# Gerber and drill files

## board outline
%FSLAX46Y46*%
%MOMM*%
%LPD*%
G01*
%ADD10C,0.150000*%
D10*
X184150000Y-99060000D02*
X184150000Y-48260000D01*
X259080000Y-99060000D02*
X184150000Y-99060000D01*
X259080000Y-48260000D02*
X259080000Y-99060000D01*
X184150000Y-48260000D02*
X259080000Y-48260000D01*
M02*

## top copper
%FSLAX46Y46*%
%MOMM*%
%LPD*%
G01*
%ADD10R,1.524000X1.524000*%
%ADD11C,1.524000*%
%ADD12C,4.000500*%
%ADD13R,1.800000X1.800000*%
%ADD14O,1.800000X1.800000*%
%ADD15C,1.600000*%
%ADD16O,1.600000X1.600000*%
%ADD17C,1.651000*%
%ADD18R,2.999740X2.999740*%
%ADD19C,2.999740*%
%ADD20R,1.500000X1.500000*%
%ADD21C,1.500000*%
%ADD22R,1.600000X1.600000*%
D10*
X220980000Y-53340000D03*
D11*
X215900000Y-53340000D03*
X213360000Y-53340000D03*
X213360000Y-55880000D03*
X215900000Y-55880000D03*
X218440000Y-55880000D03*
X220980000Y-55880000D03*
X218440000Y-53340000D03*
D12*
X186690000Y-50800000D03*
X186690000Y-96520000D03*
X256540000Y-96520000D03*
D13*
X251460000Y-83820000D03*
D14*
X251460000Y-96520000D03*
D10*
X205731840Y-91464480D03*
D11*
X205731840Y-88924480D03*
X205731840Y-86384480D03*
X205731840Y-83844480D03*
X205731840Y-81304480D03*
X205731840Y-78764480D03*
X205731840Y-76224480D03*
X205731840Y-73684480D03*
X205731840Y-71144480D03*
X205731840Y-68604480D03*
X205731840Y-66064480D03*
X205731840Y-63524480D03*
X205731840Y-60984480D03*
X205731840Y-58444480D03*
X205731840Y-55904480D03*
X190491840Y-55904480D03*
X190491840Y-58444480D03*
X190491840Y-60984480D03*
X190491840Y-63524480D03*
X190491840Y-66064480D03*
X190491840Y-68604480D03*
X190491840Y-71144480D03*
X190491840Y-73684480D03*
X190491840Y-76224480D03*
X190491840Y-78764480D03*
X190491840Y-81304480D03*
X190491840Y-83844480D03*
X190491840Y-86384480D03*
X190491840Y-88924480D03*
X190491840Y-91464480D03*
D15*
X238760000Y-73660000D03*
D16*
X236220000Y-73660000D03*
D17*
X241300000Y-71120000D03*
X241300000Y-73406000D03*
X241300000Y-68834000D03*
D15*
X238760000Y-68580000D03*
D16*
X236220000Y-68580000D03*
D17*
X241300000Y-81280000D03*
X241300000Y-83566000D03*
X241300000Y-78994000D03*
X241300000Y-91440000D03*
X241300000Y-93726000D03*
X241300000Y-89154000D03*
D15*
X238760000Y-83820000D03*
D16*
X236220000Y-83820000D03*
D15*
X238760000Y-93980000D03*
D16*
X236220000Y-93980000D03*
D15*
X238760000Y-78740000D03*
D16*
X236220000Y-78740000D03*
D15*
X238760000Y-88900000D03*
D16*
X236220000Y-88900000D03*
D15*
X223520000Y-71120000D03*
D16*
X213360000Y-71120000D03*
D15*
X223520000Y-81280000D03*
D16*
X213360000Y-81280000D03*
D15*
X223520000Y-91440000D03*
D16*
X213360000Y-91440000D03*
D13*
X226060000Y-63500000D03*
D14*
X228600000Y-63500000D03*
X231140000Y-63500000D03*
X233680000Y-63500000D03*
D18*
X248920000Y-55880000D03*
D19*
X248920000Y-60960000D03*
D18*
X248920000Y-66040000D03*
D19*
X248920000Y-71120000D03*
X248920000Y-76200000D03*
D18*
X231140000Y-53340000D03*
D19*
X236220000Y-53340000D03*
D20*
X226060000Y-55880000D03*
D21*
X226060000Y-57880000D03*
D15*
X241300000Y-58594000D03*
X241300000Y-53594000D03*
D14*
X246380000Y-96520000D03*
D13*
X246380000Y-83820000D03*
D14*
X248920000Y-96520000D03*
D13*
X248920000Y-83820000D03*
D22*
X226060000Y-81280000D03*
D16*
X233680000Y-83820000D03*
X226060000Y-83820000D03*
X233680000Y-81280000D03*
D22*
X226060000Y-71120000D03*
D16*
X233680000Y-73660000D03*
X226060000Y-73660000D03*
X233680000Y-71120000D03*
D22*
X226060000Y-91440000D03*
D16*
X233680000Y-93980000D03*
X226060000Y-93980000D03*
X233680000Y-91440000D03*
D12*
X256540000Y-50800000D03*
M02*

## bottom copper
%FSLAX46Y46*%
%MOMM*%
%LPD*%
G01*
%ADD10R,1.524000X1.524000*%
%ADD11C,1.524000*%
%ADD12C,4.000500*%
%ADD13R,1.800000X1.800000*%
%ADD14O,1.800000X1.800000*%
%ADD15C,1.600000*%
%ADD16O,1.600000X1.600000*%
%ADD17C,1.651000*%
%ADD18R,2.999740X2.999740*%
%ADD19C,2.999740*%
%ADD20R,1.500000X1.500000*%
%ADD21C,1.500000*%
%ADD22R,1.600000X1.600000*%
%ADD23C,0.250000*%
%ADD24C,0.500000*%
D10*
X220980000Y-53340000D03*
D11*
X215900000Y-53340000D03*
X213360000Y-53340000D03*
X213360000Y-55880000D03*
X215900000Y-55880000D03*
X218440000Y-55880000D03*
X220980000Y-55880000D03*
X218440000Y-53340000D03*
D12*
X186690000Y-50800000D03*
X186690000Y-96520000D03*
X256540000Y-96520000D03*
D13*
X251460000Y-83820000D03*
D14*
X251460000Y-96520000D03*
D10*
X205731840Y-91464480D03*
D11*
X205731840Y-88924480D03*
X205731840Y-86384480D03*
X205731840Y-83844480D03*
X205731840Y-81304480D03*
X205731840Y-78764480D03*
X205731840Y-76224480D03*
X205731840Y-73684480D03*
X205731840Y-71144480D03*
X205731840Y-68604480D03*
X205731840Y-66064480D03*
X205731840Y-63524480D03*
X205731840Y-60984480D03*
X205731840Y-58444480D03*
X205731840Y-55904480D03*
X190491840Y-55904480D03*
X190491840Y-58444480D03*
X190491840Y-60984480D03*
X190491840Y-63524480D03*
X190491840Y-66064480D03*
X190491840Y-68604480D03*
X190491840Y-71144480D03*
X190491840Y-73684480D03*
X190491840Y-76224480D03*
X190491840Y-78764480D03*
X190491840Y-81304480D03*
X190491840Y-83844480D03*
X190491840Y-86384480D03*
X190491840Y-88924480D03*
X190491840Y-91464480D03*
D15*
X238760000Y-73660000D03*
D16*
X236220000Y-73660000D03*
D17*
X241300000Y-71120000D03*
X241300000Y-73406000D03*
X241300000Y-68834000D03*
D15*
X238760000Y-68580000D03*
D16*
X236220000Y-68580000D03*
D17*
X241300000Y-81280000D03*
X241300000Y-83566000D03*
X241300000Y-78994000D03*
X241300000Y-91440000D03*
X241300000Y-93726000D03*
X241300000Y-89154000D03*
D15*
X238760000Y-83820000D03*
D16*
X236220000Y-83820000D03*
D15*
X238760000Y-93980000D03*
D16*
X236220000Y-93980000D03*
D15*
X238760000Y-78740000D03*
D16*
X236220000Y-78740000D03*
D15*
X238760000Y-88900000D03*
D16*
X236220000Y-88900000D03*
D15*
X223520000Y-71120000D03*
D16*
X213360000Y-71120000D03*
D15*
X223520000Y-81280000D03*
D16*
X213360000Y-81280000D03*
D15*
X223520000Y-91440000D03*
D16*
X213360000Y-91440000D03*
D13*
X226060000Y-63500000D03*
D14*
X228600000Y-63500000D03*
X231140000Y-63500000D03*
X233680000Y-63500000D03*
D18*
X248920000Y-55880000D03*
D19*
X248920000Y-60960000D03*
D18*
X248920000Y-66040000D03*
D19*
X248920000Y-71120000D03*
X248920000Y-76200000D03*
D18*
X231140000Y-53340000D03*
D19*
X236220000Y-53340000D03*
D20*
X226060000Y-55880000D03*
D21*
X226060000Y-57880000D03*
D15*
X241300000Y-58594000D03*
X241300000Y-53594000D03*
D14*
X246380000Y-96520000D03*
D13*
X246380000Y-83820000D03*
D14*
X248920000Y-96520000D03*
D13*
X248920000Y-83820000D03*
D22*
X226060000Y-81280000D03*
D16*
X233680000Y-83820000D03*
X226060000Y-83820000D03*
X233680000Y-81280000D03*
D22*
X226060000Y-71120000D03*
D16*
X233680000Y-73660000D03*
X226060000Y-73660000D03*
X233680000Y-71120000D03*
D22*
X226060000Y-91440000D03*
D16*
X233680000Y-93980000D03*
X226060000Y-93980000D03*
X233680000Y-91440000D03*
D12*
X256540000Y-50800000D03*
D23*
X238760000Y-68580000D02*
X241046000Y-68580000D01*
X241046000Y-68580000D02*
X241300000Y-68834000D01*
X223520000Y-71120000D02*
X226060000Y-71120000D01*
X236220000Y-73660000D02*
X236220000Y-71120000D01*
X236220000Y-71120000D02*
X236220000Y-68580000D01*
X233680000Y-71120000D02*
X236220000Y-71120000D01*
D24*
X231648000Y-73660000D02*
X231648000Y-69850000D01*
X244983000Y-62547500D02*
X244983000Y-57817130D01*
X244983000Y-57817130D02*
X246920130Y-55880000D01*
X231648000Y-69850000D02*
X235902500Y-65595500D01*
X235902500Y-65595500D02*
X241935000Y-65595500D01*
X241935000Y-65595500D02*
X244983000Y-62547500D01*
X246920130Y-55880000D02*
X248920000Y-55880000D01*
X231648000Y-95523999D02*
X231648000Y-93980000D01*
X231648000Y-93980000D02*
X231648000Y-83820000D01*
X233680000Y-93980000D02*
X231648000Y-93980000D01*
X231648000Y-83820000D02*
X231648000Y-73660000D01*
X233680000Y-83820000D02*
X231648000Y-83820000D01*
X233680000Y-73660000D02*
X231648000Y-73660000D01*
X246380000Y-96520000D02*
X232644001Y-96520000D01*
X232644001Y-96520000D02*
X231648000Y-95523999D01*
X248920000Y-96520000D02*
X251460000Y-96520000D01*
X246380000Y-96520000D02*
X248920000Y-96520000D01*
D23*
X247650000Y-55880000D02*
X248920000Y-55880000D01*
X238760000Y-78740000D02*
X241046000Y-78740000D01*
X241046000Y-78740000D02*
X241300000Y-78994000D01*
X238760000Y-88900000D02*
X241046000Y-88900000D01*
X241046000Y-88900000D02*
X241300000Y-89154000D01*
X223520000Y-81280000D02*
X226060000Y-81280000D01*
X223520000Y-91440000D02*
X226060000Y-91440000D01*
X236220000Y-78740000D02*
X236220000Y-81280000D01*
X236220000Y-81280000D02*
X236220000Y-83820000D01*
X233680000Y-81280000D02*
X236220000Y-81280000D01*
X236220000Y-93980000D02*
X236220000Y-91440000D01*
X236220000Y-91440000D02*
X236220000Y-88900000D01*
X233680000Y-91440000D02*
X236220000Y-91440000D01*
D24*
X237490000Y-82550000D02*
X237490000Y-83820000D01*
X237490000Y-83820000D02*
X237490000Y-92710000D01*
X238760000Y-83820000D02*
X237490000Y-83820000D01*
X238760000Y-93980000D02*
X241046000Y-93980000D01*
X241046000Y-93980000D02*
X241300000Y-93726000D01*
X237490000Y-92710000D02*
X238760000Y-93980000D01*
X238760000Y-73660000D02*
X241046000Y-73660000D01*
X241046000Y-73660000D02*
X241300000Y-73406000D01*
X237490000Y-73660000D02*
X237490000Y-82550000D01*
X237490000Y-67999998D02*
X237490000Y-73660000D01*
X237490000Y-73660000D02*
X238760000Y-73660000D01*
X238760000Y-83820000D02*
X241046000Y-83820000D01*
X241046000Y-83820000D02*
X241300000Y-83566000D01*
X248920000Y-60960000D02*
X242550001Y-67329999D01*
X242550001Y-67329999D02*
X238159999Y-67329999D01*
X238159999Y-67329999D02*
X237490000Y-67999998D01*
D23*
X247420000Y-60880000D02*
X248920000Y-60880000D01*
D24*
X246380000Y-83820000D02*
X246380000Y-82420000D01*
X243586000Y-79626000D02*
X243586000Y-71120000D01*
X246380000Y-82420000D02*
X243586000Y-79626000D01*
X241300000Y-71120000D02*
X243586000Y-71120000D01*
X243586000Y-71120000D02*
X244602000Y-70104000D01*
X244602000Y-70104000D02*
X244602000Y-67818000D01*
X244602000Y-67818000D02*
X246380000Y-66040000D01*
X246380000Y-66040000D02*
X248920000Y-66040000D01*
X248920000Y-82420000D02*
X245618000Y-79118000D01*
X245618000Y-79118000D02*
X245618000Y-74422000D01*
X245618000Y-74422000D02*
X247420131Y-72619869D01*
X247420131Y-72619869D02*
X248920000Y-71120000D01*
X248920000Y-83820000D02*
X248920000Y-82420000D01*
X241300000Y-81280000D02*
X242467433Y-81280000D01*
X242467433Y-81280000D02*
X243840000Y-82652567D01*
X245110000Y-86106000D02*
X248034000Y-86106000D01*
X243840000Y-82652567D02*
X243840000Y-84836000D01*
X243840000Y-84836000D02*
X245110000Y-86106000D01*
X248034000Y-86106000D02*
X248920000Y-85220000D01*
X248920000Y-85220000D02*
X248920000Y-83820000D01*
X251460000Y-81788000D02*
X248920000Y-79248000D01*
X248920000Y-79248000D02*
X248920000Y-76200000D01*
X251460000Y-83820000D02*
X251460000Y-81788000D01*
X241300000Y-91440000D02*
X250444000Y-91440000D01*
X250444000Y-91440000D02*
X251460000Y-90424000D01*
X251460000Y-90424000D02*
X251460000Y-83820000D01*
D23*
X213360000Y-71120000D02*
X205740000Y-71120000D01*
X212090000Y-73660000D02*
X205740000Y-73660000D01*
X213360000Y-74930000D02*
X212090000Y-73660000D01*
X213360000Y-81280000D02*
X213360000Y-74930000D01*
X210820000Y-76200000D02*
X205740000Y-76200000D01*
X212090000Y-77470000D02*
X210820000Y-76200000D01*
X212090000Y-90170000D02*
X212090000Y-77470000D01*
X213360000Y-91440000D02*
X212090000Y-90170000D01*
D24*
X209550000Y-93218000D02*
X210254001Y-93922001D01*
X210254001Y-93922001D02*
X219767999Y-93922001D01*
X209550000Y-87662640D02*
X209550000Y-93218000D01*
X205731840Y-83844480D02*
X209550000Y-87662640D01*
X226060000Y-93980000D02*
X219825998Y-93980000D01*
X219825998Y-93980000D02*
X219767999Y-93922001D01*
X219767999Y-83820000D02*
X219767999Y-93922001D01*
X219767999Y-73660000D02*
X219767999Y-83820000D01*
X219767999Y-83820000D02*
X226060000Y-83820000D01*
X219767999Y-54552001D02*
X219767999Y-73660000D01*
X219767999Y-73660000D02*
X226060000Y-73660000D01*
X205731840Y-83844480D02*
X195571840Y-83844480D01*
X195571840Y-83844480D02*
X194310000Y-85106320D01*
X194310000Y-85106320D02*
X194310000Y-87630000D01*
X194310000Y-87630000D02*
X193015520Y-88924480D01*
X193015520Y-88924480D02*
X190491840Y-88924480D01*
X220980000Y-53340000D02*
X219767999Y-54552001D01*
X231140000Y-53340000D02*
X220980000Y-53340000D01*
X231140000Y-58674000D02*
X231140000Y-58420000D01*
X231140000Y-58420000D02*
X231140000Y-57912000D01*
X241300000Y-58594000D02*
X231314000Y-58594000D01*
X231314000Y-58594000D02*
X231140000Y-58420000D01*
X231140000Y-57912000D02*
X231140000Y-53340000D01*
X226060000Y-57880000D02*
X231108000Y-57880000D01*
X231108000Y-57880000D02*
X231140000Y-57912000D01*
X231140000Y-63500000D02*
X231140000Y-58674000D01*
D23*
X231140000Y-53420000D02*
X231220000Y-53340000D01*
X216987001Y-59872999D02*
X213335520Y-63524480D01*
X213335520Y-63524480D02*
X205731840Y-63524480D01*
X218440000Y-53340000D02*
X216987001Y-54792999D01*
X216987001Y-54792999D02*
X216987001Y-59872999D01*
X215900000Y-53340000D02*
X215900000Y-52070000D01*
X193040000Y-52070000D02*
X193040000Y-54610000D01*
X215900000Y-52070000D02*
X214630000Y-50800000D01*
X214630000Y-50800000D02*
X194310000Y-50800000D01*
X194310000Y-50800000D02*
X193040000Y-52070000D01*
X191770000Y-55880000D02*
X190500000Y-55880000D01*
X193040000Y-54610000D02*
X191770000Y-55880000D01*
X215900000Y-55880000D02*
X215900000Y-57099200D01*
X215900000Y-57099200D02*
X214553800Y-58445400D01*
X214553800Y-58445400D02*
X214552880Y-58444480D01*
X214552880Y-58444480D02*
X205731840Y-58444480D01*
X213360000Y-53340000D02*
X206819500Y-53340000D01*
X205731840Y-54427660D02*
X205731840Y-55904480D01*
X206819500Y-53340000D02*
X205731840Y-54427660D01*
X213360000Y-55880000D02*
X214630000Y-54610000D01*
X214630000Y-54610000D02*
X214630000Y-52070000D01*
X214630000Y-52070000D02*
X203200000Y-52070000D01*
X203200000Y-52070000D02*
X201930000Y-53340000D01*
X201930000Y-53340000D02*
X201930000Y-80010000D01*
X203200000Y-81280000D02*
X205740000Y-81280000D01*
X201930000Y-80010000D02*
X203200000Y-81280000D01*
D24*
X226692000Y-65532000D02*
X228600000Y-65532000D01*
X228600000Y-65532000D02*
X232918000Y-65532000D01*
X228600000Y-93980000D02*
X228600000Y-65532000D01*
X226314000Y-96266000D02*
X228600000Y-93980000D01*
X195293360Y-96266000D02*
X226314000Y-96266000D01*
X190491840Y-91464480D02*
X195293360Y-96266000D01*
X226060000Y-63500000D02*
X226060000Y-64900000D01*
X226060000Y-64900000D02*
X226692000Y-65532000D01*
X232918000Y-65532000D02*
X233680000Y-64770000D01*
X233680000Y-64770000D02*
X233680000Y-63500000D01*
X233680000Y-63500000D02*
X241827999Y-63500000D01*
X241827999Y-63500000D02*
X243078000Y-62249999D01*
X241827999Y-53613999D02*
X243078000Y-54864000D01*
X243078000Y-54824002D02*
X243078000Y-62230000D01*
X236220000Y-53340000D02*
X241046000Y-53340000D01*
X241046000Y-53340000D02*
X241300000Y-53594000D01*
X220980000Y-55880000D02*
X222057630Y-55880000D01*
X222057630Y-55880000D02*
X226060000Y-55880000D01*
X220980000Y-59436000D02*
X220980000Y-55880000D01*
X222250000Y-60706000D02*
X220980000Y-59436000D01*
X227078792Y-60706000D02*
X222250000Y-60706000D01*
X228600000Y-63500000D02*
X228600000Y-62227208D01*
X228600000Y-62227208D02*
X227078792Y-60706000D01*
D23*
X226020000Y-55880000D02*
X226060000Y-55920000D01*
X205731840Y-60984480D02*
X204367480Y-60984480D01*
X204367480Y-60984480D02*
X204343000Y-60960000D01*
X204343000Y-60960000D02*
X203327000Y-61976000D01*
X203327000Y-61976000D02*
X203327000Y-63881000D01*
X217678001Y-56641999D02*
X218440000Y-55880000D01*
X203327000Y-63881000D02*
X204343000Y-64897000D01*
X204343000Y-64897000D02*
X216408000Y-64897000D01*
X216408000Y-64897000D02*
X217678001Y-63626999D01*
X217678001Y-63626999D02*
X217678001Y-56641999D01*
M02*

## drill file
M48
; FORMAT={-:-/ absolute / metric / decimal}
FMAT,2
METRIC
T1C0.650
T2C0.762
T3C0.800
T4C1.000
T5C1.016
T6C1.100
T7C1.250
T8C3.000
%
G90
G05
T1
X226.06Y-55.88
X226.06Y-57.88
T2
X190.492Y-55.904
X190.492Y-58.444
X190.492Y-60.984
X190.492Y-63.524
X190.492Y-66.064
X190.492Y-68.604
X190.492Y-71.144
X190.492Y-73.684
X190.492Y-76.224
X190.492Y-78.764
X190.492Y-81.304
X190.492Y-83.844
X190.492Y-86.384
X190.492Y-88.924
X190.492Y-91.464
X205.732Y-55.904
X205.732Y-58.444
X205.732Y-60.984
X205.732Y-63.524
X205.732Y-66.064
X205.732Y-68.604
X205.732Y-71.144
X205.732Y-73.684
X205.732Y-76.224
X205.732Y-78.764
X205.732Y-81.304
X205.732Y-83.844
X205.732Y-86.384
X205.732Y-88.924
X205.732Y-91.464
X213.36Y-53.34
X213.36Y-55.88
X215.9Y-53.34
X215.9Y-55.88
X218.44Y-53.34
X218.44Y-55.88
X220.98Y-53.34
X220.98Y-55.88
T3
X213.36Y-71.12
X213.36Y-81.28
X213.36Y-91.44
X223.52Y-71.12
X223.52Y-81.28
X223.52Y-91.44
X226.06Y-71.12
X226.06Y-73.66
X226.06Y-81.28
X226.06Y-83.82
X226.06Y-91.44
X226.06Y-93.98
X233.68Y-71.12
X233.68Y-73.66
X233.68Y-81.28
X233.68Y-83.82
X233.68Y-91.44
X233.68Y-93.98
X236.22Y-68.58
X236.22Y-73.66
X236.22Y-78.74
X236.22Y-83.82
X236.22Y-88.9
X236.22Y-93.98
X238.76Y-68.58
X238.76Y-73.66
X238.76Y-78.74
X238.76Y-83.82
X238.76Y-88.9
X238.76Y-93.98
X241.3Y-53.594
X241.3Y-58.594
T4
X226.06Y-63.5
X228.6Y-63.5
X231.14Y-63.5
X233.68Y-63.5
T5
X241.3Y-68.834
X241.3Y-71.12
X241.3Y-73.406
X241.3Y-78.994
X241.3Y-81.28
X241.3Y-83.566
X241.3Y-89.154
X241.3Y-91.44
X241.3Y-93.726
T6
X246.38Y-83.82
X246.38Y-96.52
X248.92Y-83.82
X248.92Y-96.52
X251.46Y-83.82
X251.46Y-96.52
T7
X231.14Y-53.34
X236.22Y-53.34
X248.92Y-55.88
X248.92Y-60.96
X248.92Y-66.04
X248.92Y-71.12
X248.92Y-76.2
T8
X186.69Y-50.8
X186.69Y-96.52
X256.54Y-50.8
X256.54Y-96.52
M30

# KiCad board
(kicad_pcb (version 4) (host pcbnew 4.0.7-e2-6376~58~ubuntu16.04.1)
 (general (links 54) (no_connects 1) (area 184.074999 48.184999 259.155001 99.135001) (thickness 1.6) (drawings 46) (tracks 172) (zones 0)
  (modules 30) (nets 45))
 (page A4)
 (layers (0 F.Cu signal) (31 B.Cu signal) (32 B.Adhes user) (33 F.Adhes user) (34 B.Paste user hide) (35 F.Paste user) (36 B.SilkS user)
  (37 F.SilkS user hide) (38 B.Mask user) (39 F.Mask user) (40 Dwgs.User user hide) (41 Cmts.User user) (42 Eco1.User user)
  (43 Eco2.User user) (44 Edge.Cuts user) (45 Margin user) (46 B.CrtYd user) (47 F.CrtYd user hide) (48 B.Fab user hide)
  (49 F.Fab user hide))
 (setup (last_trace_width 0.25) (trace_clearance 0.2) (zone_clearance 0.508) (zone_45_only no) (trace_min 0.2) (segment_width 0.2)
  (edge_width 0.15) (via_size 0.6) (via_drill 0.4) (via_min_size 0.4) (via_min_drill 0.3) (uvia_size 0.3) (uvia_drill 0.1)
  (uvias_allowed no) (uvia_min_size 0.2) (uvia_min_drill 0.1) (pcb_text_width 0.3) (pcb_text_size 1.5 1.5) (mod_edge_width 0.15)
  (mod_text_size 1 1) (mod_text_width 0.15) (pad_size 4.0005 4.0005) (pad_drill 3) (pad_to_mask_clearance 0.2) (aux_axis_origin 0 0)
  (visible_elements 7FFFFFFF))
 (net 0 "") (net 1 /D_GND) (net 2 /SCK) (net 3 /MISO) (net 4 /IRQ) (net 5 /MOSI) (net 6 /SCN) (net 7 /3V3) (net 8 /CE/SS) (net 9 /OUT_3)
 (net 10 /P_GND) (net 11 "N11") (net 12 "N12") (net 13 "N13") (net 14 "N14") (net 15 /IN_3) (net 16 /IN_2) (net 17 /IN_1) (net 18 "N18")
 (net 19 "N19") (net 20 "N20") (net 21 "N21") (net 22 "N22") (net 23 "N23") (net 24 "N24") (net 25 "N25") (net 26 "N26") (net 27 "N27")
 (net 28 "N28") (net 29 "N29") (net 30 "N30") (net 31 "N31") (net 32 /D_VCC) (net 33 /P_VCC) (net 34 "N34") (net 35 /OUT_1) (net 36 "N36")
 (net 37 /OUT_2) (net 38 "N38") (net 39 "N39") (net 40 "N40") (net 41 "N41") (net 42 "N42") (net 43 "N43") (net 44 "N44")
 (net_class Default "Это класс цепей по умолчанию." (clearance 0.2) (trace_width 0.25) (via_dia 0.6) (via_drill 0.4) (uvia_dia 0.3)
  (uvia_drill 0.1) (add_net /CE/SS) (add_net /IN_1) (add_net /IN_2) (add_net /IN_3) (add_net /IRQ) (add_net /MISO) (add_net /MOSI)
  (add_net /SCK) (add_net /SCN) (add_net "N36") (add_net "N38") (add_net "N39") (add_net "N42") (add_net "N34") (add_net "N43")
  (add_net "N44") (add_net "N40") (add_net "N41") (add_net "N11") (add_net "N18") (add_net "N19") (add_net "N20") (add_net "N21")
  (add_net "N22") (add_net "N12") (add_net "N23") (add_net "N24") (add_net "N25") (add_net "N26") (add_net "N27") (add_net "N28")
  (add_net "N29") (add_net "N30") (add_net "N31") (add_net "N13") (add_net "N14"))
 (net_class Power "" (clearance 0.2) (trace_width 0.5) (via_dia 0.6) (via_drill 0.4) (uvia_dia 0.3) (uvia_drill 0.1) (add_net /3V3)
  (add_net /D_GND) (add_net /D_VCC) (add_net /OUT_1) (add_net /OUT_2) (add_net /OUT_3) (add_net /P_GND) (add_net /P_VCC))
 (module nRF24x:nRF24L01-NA (layer F.Cu) (at 215.265 67.31)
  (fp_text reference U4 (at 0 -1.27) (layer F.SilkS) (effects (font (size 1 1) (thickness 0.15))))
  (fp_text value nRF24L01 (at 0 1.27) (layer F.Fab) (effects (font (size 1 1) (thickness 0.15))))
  (pad 1 thru_hole rect (at 5.715 -13.97) (size 1.524 1.524) (drill 0.762) (layers *.Cu *.Mask) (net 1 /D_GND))
  (pad 5 thru_hole circle (at 0.635 -13.97) (size 1.524 1.524) (drill 0.762) (layers *.Cu *.Mask) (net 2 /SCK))
  (pad 7 thru_hole circle (at -1.905 -13.97) (size 1.524 1.524) (drill 0.762) (layers *.Cu *.Mask) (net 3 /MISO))
  (pad 8 thru_hole circle (at -1.905 -11.43) (size 1.524 1.524) (drill 0.762) (layers *.Cu *.Mask) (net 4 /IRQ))
  (pad 6 thru_hole circle (at 0.635 -11.43) (size 1.524 1.524) (drill 0.762) (layers *.Cu *.Mask) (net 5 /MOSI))
  (pad 4 thru_hole circle (at 3.175 -11.43) (size 1.524 1.524) (drill 0.762) (layers *.Cu *.Mask) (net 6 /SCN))
  (pad 2 thru_hole circle (at 5.715 -11.43) (size 1.524 1.524) (drill 0.762) (layers *.Cu *.Mask) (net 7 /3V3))
  (pad 3 thru_hole circle (at 3.175 -13.97) (size 1.524 1.524) (drill 0.762) (layers *.Cu *.Mask) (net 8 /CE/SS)))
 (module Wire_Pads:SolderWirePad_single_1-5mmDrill (layer F.Cu) (at 186.69 50.8)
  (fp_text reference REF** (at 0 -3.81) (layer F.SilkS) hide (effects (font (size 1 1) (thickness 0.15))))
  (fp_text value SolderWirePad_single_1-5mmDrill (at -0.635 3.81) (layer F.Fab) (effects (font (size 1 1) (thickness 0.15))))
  (pad 1 thru_hole circle (at 0 0) (size 4.0005 4.0005) (drill 3) (layers *.Cu *.Mask)))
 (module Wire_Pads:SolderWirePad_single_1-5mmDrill (layer F.Cu) (at 186.69 96.52)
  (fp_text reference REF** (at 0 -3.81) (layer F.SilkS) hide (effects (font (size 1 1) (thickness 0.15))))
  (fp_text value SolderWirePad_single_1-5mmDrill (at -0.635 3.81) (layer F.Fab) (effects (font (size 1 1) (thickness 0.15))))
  (pad 1 thru_hole circle (at 0 0) (size 4.0005 4.0005) (drill 3) (layers *.Cu *.Mask)))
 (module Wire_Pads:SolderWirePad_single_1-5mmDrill (layer F.Cu) (at 256.54 96.52)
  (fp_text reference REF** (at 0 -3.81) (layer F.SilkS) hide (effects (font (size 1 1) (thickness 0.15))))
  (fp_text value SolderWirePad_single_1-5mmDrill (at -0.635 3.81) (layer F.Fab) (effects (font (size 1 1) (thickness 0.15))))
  (pad 1 thru_hole circle (at 0 0) (size 4.0005 4.0005) (drill 3) (layers *.Cu *.Mask)))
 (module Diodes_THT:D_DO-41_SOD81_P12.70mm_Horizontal (layer F.Cu) (at 251.46 83.82 270)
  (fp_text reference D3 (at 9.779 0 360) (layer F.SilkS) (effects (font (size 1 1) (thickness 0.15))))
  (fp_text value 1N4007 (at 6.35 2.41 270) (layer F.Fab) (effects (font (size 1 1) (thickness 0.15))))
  (pad 1 thru_hole rect (at 0 0 270) (size 1.8 1.8) (drill 1.1) (layers *.Cu *.Mask) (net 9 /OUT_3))
  (pad 2 thru_hole oval (at 12.7 0 270) (size 1.8 1.8) (drill 1.1) (layers *.Cu *.Mask) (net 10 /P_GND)))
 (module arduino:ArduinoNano (layer F.Cu) (at 198.12 73.66)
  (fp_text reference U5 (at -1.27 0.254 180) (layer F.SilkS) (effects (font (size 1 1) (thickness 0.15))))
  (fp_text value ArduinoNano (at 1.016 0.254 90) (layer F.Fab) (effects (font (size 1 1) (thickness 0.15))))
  (pad 1 thru_hole rect (at 7.61184 17.80448) (size 1.524 1.524) (drill 0.762) (layers *.Cu *.Mask) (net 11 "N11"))
  (pad 2 thru_hole circle (at 7.61184 15.26448) (size 1.524 1.524) (drill 0.762) (layers *.Cu *.Mask) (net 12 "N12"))
  (pad 3 thru_hole circle (at 7.61184 12.72448) (size 1.524 1.524) (drill 0.762) (layers *.Cu *.Mask) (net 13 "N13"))
  (pad 4 thru_hole circle (at 7.61184 10.18448) (size 1.524 1.524) (drill 0.762) (layers *.Cu *.Mask) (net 1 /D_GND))
  (pad 5 thru_hole circle (at 7.61184 7.64448) (size 1.524 1.524) (drill 0.762) (layers *.Cu *.Mask) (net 4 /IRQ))
  (pad 6 thru_hole circle (at 7.61184 5.10448) (size 1.524 1.524) (drill 0.762) (layers *.Cu *.Mask) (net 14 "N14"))
  (pad 7 thru_hole circle (at 7.61184 2.56448) (size 1.524 1.524) (drill 0.762) (layers *.Cu *.Mask) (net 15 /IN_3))
  (pad 8 thru_hole circle (at 7.61184 0.02448) (size 1.524 1.524) (drill 0.762) (layers *.Cu *.Mask) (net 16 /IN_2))
  (pad 9 thru_hole circle (at 7.61184 -2.51552) (size 1.524 1.524) (drill 0.762) (layers *.Cu *.Mask) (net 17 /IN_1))
  (pad 10 thru_hole circle (at 7.61184 -5.05552) (size 1.524 1.524) (drill 0.762) (layers *.Cu *.Mask) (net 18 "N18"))
  (pad 11 thru_hole circle (at 7.61184 -7.59552) (size 1.524 1.524) (drill 0.762) (layers *.Cu *.Mask) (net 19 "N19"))
  (pad 12 thru_hole circle (at 7.61184 -10.13552) (size 1.524 1.524) (drill 0.762) (layers *.Cu *.Mask) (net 8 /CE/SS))
  (pad 13 thru_hole circle (at 7.61184 -12.67552) (size 1.524 1.524) (drill 0.762) (layers *.Cu *.Mask) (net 6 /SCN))
  (pad 14 thru_hole circle (at 7.61184 -15.21552) (size 1.524 1.524) (drill 0.762) (layers *.Cu *.Mask) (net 5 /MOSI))
  (pad 15 thru_hole circle (at 7.61184 -17.75552) (size 1.524 1.524) (drill 0.762) (layers *.Cu *.Mask) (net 3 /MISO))
  (pad 16 thru_hole circle (at -7.62816 -17.75552) (size 1.524 1.524) (drill 0.762) (layers *.Cu *.Mask) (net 2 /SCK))
  (pad 17 thru_hole circle (at -7.62816 -15.21552) (size 1.524 1.524) (drill 0.762) (layers *.Cu *.Mask) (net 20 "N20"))
  (pad 18 thru_hole circle (at -7.62816 -12.67552) (size 1.524 1.524) (drill 0.762) (layers *.Cu *.Mask) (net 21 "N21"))
  (pad 19 thru_hole circle (at -7.62816 -10.13552) (size 1.524 1.524) (drill 0.762) (layers *.Cu *.Mask) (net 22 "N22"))
  (pad 20 thru_hole circle (at -7.62816 -7.59552) (size 1.524 1.524) (drill 0.762) (layers *.Cu *.Mask) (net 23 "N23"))
  (pad 21 thru_hole circle (at -7.62816 -5.05552) (size 1.524 1.524) (drill 0.762) (layers *.Cu *.Mask) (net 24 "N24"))
  (pad 22 thru_hole circle (at -7.62816 -2.51552) (size 1.524 1.524) (drill 0.762) (layers *.Cu *.Mask) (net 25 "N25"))
  (pad 23 thru_hole circle (at -7.62816 0.02448) (size 1.524 1.524) (drill 0.762) (layers *.Cu *.Mask) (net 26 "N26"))
  (pad 24 thru_hole circle (at -7.62816 2.56448) (size 1.524 1.524) (drill 0.762) (layers *.Cu *.Mask) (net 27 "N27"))
  (pad 25 thru_hole circle (at -7.62816 5.10448) (size 1.524 1.524) (drill 0.762) (layers *.Cu *.Mask) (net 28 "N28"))
  (pad 26 thru_hole circle (at -7.62816 7.64448) (size 1.524 1.524) (drill 0.762) (layers *.Cu *.Mask) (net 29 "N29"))
  (pad 27 thru_hole circle (at -7.62816 10.18448) (size 1.524 1.524) (drill 0.762) (layers *.Cu *.Mask) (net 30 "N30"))
  (pad 28 thru_hole circle (at -7.62816 12.72448) (size 1.524 1.524) (drill 0.762) (layers *.Cu *.Mask) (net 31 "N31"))
  (pad 29 thru_hole circle (at -7.62816 15.26448) (size 1.524 1.524) (drill 0.762) (layers *.Cu *.Mask) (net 1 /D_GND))
  (pad 30 thru_hole circle (at -7.62816 17.80448) (size 1.524 1.524) (drill 0.762) (layers *.Cu *.Mask) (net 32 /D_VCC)))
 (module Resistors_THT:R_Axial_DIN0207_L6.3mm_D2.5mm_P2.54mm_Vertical (layer F.Cu) (at 238.76 73.66 180)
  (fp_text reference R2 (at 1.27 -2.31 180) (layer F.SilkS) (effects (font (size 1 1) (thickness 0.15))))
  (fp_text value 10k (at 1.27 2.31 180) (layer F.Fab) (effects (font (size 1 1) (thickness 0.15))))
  (pad 1 thru_hole circle (at 0 0 180) (size 1.6 1.6) (drill 0.8) (layers *.Cu *.Mask) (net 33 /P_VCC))
  (pad 2 thru_hole oval (at 2.54 0 180) (size 1.6 1.6) (drill 0.8) (layers *.Cu *.Mask) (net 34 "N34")))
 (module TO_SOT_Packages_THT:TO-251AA (layer F.Cu) (at 241.3 68.834 270)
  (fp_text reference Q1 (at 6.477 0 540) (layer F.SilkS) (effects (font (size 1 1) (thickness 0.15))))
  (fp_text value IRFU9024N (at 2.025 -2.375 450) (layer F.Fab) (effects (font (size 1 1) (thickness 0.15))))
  (pad 2 thru_hole circle (at 2.286 0 90) (size 1.651 1.651) (drill 1.016) (layers *.Cu *.Mask) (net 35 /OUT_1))
  (pad 3 thru_hole circle (at 4.572 0 90) (size 1.651 1.651) (drill 1.016) (layers *.Cu *.Mask) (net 33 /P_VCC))
  (pad 1 thru_hole circle (at 0 0 90) (size 1.651 1.651) (drill 1.016) (layers *.Cu *.Mask) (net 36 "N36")))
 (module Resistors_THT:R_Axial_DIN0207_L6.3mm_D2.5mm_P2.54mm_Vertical (layer F.Cu) (at 238.76 68.58 180)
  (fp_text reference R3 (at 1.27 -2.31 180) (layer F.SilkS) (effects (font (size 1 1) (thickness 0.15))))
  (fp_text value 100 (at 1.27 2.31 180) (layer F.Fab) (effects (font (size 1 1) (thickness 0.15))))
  (pad 1 thru_hole circle (at 0 0 180) (size 1.6 1.6) (drill 0.8) (layers *.Cu *.Mask) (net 36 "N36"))
  (pad 2 thru_hole oval (at 2.54 0 180) (size 1.6 1.6) (drill 0.8) (layers *.Cu *.Mask) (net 34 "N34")))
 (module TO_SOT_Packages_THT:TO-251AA (layer F.Cu) (at 241.3 78.994 270)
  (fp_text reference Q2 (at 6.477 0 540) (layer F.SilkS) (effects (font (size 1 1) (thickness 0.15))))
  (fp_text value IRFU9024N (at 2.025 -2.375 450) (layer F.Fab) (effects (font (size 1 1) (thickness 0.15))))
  (pad 2 thru_hole circle (at 2.286 0 90) (size 1.651 1.651) (drill 1.016) (layers *.Cu *.Mask) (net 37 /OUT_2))
  (pad 3 thru_hole circle (at 4.572 0 90) (size 1.651 1.651) (drill 1.016) (layers *.Cu *.Mask) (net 33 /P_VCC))
  (pad 1 thru_hole circle (at 0 0 90) (size 1.651 1.651) (drill 1.016) (layers *.Cu *.Mask) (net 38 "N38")))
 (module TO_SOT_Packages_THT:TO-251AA (layer F.Cu) (at 241.3 89.154 270)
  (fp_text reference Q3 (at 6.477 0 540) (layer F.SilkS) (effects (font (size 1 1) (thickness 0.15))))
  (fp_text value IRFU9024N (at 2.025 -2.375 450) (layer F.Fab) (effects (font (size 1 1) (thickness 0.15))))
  (pad 2 thru_hole circle (at 2.286 0 90) (size 1.651 1.651) (drill 1.016) (layers *.Cu *.Mask) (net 9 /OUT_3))
  (pad 3 thru_hole circle (at 4.572 0 90) (size 1.651 1.651) (drill 1.016) (layers *.Cu *.Mask) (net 33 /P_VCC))
  (pad 1 thru_hole circle (at 0 0 90) (size 1.651 1.651) (drill 1.016) (layers *.Cu *.Mask) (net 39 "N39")))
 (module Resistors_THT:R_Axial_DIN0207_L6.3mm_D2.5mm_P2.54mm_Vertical (layer F.Cu) (at 238.76 83.82 180)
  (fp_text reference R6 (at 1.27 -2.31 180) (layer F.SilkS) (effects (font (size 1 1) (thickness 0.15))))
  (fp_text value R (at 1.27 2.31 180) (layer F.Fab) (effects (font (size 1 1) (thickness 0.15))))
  (pad 1 thru_hole circle (at 0 0 180) (size 1.6 1.6) (drill 0.8) (layers *.Cu *.Mask) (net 33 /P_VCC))
  (pad 2 thru_hole oval (at 2.54 0 180) (size 1.6 1.6) (drill 0.8) (layers *.Cu *.Mask) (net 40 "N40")))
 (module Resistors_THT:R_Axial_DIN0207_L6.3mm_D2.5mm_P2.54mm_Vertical (layer F.Cu) (at 238.76 93.98 180)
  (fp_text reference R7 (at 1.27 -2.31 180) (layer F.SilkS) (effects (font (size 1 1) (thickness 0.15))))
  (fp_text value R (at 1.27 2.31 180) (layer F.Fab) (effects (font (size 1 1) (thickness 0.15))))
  (pad 1 thru_hole circle (at 0 0 180) (size 1.6 1.6) (drill 0.8) (layers *.Cu *.Mask) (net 33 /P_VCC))
  (pad 2 thru_hole oval (at 2.54 0 180) (size 1.6 1.6) (drill 0.8) (layers *.Cu *.Mask) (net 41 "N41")))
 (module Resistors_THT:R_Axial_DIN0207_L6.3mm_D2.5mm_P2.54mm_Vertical (layer F.Cu) (at 238.76 78.74 180)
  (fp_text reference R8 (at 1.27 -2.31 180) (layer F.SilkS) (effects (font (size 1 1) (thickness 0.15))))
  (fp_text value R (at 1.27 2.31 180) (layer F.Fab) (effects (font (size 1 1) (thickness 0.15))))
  (pad 1 thru_hole circle (at 0 0 180) (size 1.6 1.6) (drill 0.8) (layers *.Cu *.Mask) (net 38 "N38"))
  (pad 2 thru_hole oval (at 2.54 0 180) (size 1.6 1.6) (drill 0.8) (layers *.Cu *.Mask) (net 40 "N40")))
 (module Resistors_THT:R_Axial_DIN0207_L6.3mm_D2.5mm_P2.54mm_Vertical (layer F.Cu) (at 238.76 88.9 180)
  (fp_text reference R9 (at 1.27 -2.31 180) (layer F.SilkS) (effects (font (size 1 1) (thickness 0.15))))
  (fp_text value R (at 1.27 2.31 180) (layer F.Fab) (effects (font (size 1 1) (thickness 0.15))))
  (pad 1 thru_hole circle (at 0 0 180) (size 1.6 1.6) (drill 0.8) (layers *.Cu *.Mask) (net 39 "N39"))
  (pad 2 thru_hole oval (at 2.54 0 180) (size 1.6 1.6) (drill 0.8) (layers *.Cu *.Mask) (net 41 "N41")))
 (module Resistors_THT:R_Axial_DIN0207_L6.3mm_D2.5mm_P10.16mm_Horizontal (layer F.Cu) (at 223.52 71.12 180)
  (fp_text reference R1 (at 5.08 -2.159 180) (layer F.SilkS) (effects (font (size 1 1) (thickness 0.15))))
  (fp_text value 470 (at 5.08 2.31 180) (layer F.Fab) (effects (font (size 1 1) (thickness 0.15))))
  (pad 1 thru_hole circle (at 0 0 180) (size 1.6 1.6) (drill 0.8) (layers *.Cu *.Mask) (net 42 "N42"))
  (pad 2 thru_hole oval (at 10.16 0 180) (size 1.6 1.6) (drill 0.8) (layers *.Cu *.Mask) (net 17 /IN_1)))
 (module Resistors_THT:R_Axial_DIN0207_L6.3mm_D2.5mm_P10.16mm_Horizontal (layer F.Cu) (at 223.52 81.28 180)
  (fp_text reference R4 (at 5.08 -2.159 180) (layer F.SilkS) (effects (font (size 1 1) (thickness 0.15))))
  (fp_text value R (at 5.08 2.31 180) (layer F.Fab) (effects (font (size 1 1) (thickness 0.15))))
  (pad 1 thru_hole circle (at 0 0 180) (size 1.6 1.6) (drill 0.8) (layers *.Cu *.Mask) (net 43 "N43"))
  (pad 2 thru_hole oval (at 10.16 0 180) (size 1.6 1.6) (drill 0.8) (layers *.Cu *.Mask) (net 16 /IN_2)))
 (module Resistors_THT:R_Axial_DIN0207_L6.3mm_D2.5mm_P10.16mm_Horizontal (layer F.Cu) (at 223.52 91.44 180)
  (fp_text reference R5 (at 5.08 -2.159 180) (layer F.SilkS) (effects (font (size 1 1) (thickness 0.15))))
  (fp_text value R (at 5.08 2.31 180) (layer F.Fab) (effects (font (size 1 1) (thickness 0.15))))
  (pad 1 thru_hole circle (at 0 0 180) (size 1.6 1.6) (drill 0.8) (layers *.Cu *.Mask) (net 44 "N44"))
  (pad 2 thru_hole oval (at 10.16 0 180) (size 1.6 1.6) (drill 0.8) (layers *.Cu *.Mask) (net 15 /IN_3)))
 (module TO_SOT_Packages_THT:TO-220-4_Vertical (layer F.Cu) (at 226.06 63.5)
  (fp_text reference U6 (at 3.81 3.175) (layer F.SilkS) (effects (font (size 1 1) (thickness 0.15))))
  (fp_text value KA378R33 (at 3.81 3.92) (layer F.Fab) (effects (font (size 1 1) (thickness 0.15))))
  (pad 1 thru_hole rect (at 0 0) (size 1.8 1.8) (drill 1) (layers *.Cu *.Mask) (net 32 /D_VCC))
  (pad 2 thru_hole oval (at 2.54 0) (size 1.8 1.8) (drill 1) (layers *.Cu *.Mask) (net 7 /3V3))
  (pad 3 thru_hole oval (at 5.08 0) (size 1.8 1.8) (drill 1) (layers *.Cu *.Mask) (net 1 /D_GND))
  (pad 4 thru_hole oval (at 7.62 0) (size 1.8 1.8) (drill 1) (layers *.Cu *.Mask) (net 32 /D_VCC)))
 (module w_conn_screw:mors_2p (layer F.Cu) (at 248.92 58.42 270)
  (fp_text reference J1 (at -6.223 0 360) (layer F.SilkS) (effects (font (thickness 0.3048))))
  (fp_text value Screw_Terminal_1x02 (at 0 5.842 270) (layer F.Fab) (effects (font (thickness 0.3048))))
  (pad 1 thru_hole rect (at -2.54 0 270) (size 2.99974 2.99974) (drill 1.24968) (layers *.Cu *.Mask F.SilkS) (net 10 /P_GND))
  (pad 2 thru_hole circle (at 2.54 0 270) (size 2.99974 2.99974) (drill 1.24968) (layers *.Cu *.Mask F.SilkS) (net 33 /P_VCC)))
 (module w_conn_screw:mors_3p (layer F.Cu) (at 248.92 71.12 270)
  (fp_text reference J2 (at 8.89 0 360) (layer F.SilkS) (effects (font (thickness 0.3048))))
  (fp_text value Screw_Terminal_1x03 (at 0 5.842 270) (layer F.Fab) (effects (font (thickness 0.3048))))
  (pad 1 thru_hole rect (at -5.08 0 270) (size 2.99974 2.99974) (drill 1.24968) (layers *.Cu *.Mask F.SilkS) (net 35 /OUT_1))
  (pad 2 thru_hole circle (at 0 0 270) (size 2.99974 2.99974) (drill 1.24968) (layers *.Cu *.Mask F.SilkS) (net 37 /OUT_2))
  (pad 3 thru_hole circle (at 5.08 0 270) (size 2.99974 2.99974) (drill 1.24968) (layers *.Cu *.Mask F.SilkS) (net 9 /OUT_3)))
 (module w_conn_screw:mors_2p (layer F.Cu) (at 233.68 53.34)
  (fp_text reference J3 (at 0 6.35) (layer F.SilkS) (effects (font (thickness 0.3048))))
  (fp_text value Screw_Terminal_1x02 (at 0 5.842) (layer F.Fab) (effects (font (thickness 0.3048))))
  (pad 1 thru_hole rect (at -2.54 0) (size 2.99974 2.99974) (drill 1.24968) (layers *.Cu *.Mask F.SilkS) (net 1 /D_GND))
  (pad 2 thru_hole circle (at 2.54 0) (size 2.99974 2.99974) (drill 1.24968) (layers *.Cu *.Mask F.SilkS) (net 32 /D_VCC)))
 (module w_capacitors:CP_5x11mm (layer F.Cu) (at 226.06 56.88 180)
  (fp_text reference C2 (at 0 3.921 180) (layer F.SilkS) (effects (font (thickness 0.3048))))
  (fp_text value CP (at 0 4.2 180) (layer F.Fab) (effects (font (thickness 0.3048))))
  (pad 1 thru_hole rect (at 0 1 180) (size 1.5 1.5) (drill 0.65) (layers *.Cu *.Mask F.SilkS) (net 7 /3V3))
  (pad 2 thru_hole circle (at 0 -1 180) (size 1.5 1.5) (drill 0.65) (layers *.Cu *.Mask F.SilkS) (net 1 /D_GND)))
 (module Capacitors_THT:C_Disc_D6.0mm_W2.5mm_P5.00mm (layer F.Cu) (at 241.3 53.594 270)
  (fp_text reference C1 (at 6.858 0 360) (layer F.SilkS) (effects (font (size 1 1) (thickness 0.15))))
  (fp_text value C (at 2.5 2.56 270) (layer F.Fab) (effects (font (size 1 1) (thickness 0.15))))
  (pad 2 thru_hole circle (at 5 0 270) (size 1.6 1.6) (drill 0.8) (layers *.Cu *.Mask) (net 1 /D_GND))
  (pad 1 thru_hole circle (at 0 0 270) (size 1.6 1.6) (drill 0.8) (layers *.Cu *.Mask) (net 32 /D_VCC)))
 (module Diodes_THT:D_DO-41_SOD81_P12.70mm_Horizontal (layer F.Cu) (at 246.38 83.82 270)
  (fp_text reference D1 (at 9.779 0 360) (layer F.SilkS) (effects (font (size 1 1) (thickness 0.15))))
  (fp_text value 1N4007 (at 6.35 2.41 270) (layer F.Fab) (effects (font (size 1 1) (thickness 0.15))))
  (pad 2 thru_hole oval (at 12.7 0 270) (size 1.8 1.8) (drill 1.1) (layers *.Cu *.Mask) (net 10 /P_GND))
  (pad 1 thru_hole rect (at 0 0 270) (size 1.8 1.8) (drill 1.1) (layers *.Cu *.Mask) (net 35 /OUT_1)))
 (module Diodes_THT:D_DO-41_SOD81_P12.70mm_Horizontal (layer F.Cu) (at 248.92 83.82 270)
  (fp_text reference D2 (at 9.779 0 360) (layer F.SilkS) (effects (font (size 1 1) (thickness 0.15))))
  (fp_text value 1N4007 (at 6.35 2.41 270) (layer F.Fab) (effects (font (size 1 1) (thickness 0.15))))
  (pad 2 thru_hole oval (at 12.7 0 270) (size 1.8 1.8) (drill 1.1) (layers *.Cu *.Mask) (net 10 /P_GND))
  (pad 1 thru_hole rect (at 0 0 270) (size 1.8 1.8) (drill 1.1) (layers *.Cu *.Mask) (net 37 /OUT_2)))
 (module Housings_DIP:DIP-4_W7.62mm (layer F.Cu) (at 226.06 81.28)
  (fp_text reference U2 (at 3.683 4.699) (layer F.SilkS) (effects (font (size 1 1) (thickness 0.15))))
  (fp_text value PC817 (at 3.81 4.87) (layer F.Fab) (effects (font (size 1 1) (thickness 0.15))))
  (pad 1 thru_hole rect (at 0 0) (size 1.6 1.6) (drill 0.8) (layers *.Cu *.Mask) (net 43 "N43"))
  (pad 3 thru_hole oval (at 7.62 2.54) (size 1.6 1.6) (drill 0.8) (layers *.Cu *.Mask) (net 10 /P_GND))
  (pad 2 thru_hole oval (at 0 2.54) (size 1.6 1.6) (drill 0.8) (layers *.Cu *.Mask) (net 1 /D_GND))
  (pad 4 thru_hole oval (at 7.62 0) (size 1.6 1.6) (drill 0.8) (layers *.Cu *.Mask) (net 40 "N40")))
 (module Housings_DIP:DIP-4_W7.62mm (layer F.Cu) (at 226.06 71.12)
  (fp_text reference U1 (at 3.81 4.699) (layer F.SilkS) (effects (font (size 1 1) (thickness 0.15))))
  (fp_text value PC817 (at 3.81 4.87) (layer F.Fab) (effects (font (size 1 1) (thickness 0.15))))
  (pad 1 thru_hole rect (at 0 0) (size 1.6 1.6) (drill 0.8) (layers *.Cu *.Mask) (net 42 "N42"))
  (pad 3 thru_hole oval (at 7.62 2.54) (size 1.6 1.6) (drill 0.8) (layers *.Cu *.Mask) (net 10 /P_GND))
  (pad 2 thru_hole oval (at 0 2.54) (size 1.6 1.6) (drill 0.8) (layers *.Cu *.Mask) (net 1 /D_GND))
  (pad 4 thru_hole oval (at 7.62 0) (size 1.6 1.6) (drill 0.8) (layers *.Cu *.Mask) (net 34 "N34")))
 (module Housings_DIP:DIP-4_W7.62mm (layer F.Cu) (at 226.06 91.44)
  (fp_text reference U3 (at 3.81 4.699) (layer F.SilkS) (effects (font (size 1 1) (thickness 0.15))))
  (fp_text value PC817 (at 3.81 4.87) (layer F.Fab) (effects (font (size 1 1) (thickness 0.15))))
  (pad 1 thru_hole rect (at 0 0) (size 1.6 1.6) (drill 0.8) (layers *.Cu *.Mask) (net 44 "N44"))
  (pad 3 thru_hole oval (at 7.62 2.54) (size 1.6 1.6) (drill 0.8) (layers *.Cu *.Mask) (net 10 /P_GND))
  (pad 2 thru_hole oval (at 0 2.54) (size 1.6 1.6) (drill 0.8) (layers *.Cu *.Mask) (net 1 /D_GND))
  (pad 4 thru_hole oval (at 7.62 0) (size 1.6 1.6) (drill 0.8) (layers *.Cu *.Mask) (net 41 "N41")))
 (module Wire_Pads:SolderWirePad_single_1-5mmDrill (layer F.Cu) (at 256.54 50.8)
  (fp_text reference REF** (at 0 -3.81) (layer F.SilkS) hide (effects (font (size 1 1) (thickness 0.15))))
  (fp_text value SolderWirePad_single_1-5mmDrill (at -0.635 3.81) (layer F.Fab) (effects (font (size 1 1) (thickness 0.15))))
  (pad 1 thru_hole circle (at 0 0) (size 4.0005 4.0005) (drill 3) (layers *.Cu *.Mask)))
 (gr_line (start 184.15 99.06) (end 184.15 48.26) (layer Edge.Cuts) (width 0.15))
 (gr_line (start 259.08 99.06) (end 184.15 99.06) (layer Edge.Cuts) (width 0.15))
 (gr_line (start 259.08 48.26) (end 259.08 99.06) (layer Edge.Cuts) (width 0.15))
 (gr_line (start 184.15 48.26) (end 259.08 48.26) (layer Edge.Cuts) (width 0.15))
 (segment (start 238.76 68.58) (end 241.046 68.58) (width 0.25) (layer B.Cu) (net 36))
 (segment (start 241.046 68.58) (end 241.3 68.834) (width 0.25) (layer B.Cu) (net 36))
 (segment (start 223.52 71.12) (end 226.06 71.12) (width 0.25) (layer B.Cu) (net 42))
 (segment (start 236.22 73.66) (end 236.22 71.12) (width 0.25) (layer B.Cu) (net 34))
 (segment (start 236.22 71.12) (end 236.22 68.58) (width 0.25) (layer B.Cu) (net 34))
 (segment (start 233.68 71.12) (end 236.22 71.12) (width 0.25) (layer B.Cu) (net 34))
 (segment (start 231.648 73.66) (end 231.648 69.85) (width 0.5) (layer B.Cu) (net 10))
 (segment (start 244.983 62.5475) (end 244.983 57.81713) (width 0.5) (layer B.Cu) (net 10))
 (segment (start 244.983 57.81713) (end 246.92013 55.88) (width 0.5) (layer B.Cu) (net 10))
 (segment (start 231.648 69.85) (end 235.9025 65.5955) (width 0.5) (layer B.Cu) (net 10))
 (segment (start 235.9025 65.5955) (end 241.935 65.5955) (width 0.5) (layer B.Cu) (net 10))
 (segment (start 241.935 65.5955) (end 244.983 62.5475) (width 0.5) (layer B.Cu) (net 10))
 (segment (start 246.92013 55.88) (end 248.92 55.88) (width 0.5) (layer B.Cu) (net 10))
 (segment (start 231.648 95.523999) (end 231.648 93.98) (width 0.5) (layer B.Cu) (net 10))
 (segment (start 231.648 93.98) (end 231.648 83.82) (width 0.5) (layer B.Cu) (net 10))
 (segment (start 233.68 93.98) (end 231.648 93.98) (width 0.5) (layer B.Cu) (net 10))
 (segment (start 231.648 83.82) (end 231.648 73.66) (width 0.5) (layer B.Cu) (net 10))
 (segment (start 233.68 83.82) (end 231.648 83.82) (width 0.5) (layer B.Cu) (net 10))
 (segment (start 233.68 73.66) (end 231.648 73.66) (width 0.5) (layer B.Cu) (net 10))
 (segment (start 246.38 96.52) (end 232.644001 96.52) (width 0.5) (layer B.Cu) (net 10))
 (segment (start 232.644001 96.52) (end 231.648 95.523999) (width 0.5) (layer B.Cu) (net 10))
 (segment (start 248.92 96.52) (end 251.46 96.52) (width 0.5) (layer B.Cu) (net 10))
 (segment (start 246.38 96.52) (end 248.92 96.52) (width 0.5) (layer B.Cu) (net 10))
 (segment (start 247.65 55.88) (end 248.92 55.88) (width 0.25) (layer B.Cu) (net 10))
 (segment (start 238.76 78.74) (end 241.046 78.74) (width 0.25) (layer B.Cu) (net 38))
 (segment (start 241.046 78.74) (end 241.3 78.994) (width 0.25) (layer B.Cu) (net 38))
 (segment (start 238.76 88.9) (end 241.046 88.9) (width 0.25) (layer B.Cu) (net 39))
 (segment (start 241.046 88.9) (end 241.3 89.154) (width 0.25) (layer B.Cu) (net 39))
 (segment (start 223.52 81.28) (end 226.06 81.28) (width 0.25) (layer B.Cu) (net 43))
 (segment (start 223.52 91.44) (end 226.06 91.44) (width 0.25) (layer B.Cu) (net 44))
 (segment (start 236.22 78.74) (end 236.22 81.28) (width 0.25) (layer B.Cu) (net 40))
 (segment (start 236.22 81.28) (end 236.22 83.82) (width 0.25) (layer B.Cu) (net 40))
 (segment (start 233.68 81.28) (end 236.22 81.28) (width 0.25) (layer B.Cu) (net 40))
 (segment (start 236.22 93.98) (end 236.22 91.44) (width 0.25) (layer B.Cu) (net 41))
 (segment (start 236.22 91.44) (end 236.22 88.9) (width 0.25) (layer B.Cu) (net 41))
 (segment (start 233.68 91.44) (end 236.22 91.44) (width 0.25) (layer B.Cu) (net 41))
 (segment (start 237.49 82.55) (end 237.49 83.82) (width 0.5) (layer B.Cu) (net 33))
 (segment (start 237.49 83.82) (end 237.49 92.71) (width 0.5) (layer B.Cu) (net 33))
 (segment (start 238.76 83.82) (end 237.49 83.82) (width 0.5) (layer B.Cu) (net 33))
 (segment (start 238.76 93.98) (end 241.046 93.98) (width 0.5) (layer B.Cu) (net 33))
 (segment (start 241.046 93.98) (end 241.3 93.726) (width 0.5) (layer B.Cu) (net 33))
 (segment (start 237.49 92.71) (end 238.76 93.98) (width 0.5) (layer B.Cu) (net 33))
 (segment (start 238.76 73.66) (end 241.046 73.66) (width 0.5) (layer B.Cu) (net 33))
 (segment (start 241.046 73.66) (end 241.3 73.406) (width 0.5) (layer B.Cu) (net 33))
 (segment (start 237.49 73.66) (end 237.49 82.55) (width 0.5) (layer B.Cu) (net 33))
 (segment (start 237.49 67.999998) (end 237.49 73.66) (width 0.5) (layer B.Cu) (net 33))
 (segment (start 237.49 73.66) (end 238.76 73.66) (width 0.5) (layer B.Cu) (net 33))
 (segment (start 238.76 83.82) (end 241.046 83.82) (width 0.5) (layer B.Cu) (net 33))
 (segment (start 241.046 83.82) (end 241.3 83.566) (width 0.5) (layer B.Cu) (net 33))
 (segment (start 248.92 60.96) (end 242.550001 67.329999) (width 0.5) (layer B.Cu) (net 33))
 (segment (start 242.550001 67.329999) (end 238.159999 67.329999) (width 0.5) (layer B.Cu) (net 33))
 (segment (start 238.159999 67.329999) (end 237.49 67.999998) (width 0.5) (layer B.Cu) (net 33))
 (segment (start 247.42 60.88) (end 248.92 60.88) (width 0.25) (layer B.Cu) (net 33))
 (segment (start 246.38 83.82) (end 246.38 82.42) (width 0.5) (layer B.Cu) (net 35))
 (segment (start 243.586 79.626) (end 243.586 71.12) (width 0.5) (layer B.Cu) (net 35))
 (segment (start 246.38 82.42) (end 243.586 79.626) (width 0.5) (layer B.Cu) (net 35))
 (segment (start 241.3 71.12) (end 243.586 71.12) (width 0.5) (layer B.Cu) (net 35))
 (segment (start 243.586 71.12) (end 244.602 70.104) (width 0.5) (layer B.Cu) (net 35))
 (segment (start 244.602 70.104) (end 244.602 67.818) (width 0.5) (layer B.Cu) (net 35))
 (segment (start 244.602 67.818) (end 246.38 66.04) (width 0.5) (layer B.Cu) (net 35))
 (segment (start 246.38 66.04) (end 248.92 66.04) (width 0.5) (layer B.Cu) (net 35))
 (segment (start 248.92 82.42) (end 245.618 79.118) (width 0.5) (layer B.Cu) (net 37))
 (segment (start 245.618 79.118) (end 245.618 74.422) (width 0.5) (layer B.Cu) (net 37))
 (segment (start 245.618 74.422) (end 247.420131 72.619869) (width 0.5) (layer B.Cu) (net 37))
 (segment (start 247.420131 72.619869) (end 248.92 71.12) (width 0.5) (layer B.Cu) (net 37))
 (segment (start 248.92 83.82) (end 248.92 82.42) (width 0.5) (layer B.Cu) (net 37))
 (segment (start 241.3 81.28) (end 242.467433 81.28) (width 0.5) (layer B.Cu) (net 37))
 (segment (start 242.467433 81.28) (end 243.84 82.652567) (width 0.5) (layer B.Cu) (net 37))
 (segment (start 245.11 86.106) (end 248.034 86.106) (width 0.5) (layer B.Cu) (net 37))
 (segment (start 243.84 82.652567) (end 243.84 84.836) (width 0.5) (layer B.Cu) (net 37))
 (segment (start 243.84 84.836) (end 245.11 86.106) (width 0.5) (layer B.Cu) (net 37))
 (segment (start 248.034 86.106) (end 248.92 85.22) (width 0.5) (layer B.Cu) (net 37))
 (segment (start 248.92 85.22) (end 248.92 83.82) (width 0.5) (layer B.Cu) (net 37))
 (segment (start 251.46 81.788) (end 248.92 79.248) (width 0.5) (layer B.Cu) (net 9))
 (segment (start 248.92 79.248) (end 248.92 76.2) (width 0.5) (layer B.Cu) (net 9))
 (segment (start 251.46 83.82) (end 251.46 81.788) (width 0.5) (layer B.Cu) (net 9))
 (segment (start 241.3 91.44) (end 250.444 91.44) (width 0.5) (layer B.Cu) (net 9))
 (segment (start 250.444 91.44) (end 251.46 90.424) (width 0.5) (layer B.Cu) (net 9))
 (segment (start 251.46 90.424) (end 251.46 83.82) (width 0.5) (layer B.Cu) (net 9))
 (segment (start 213.36 71.12) (end 205.74 71.12) (width 0.25) (layer B.Cu) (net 17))
 (segment (start 212.09 73.66) (end 205.74 73.66) (width 0.25) (layer B.Cu) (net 16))
 (segment (start 213.36 74.93) (end 212.09 73.66) (width 0.25) (layer B.Cu) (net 16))
 (segment (start 213.36 81.28) (end 213.36 74.93) (width 0.25) (layer B.Cu) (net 16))
 (segment (start 210.82 76.2) (end 205.74 76.2) (width 0.25) (layer B.Cu) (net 15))
 (segment (start 212.09 77.47) (end 210.82 76.2) (width 0.25) (layer B.Cu) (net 15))
 (segment (start 212.09 90.17) (end 212.09 77.47) (width 0.25) (layer B.Cu) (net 15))
 (segment (start 213.36 91.44) (end 212.09 90.17) (width 0.25) (layer B.Cu) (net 15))
 (segment (start 209.55 93.218) (end 210.254001 93.922001) (width 0.5) (layer B.Cu) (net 1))
 (segment (start 210.254001 93.922001) (end 219.767999 93.922001) (width 0.5) (layer B.Cu) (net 1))
 (segment (start 209.55 87.66264) (end 209.55 93.218) (width 0.5) (layer B.Cu) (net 1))
 (segment (start 205.73184 83.84448) (end 209.55 87.66264) (width 0.5) (layer B.Cu) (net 1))
 (segment (start 226.06 93.98) (end 219.825998 93.98) (width 0.5) (layer B.Cu) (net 1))
 (segment (start 219.825998 93.98) (end 219.767999 93.922001) (width 0.5) (layer B.Cu) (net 1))
 (segment (start 219.767999 83.82) (end 219.767999 93.922001) (width 0.5) (layer B.Cu) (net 1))
 (segment (start 219.767999 73.66) (end 219.767999 83.82) (width 0.5) (layer B.Cu) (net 1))
 (segment (start 219.767999 83.82) (end 226.06 83.82) (width 0.5) (layer B.Cu) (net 1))
 (segment (start 219.767999 54.552001) (end 219.767999 73.66) (width 0.5) (layer B.Cu) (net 1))
 (segment (start 219.767999 73.66) (end 226.06 73.66) (width 0.5) (layer B.Cu) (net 1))
 (segment (start 205.73184 83.84448) (end 195.57184 83.84448) (width 0.5) (layer B.Cu) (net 1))
 (segment (start 195.57184 83.84448) (end 194.31 85.10632) (width 0.5) (layer B.Cu) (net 1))
 (segment (start 194.31 85.10632) (end 194.31 87.63) (width 0.5) (layer B.Cu) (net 1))
 (segment (start 194.31 87.63) (end 193.01552 88.92448) (width 0.5) (layer B.Cu) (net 1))
 (segment (start 193.01552 88.92448) (end 190.49184 88.92448) (width 0.5) (layer B.Cu) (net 1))
 (segment (start 220.98 53.34) (end 219.767999 54.552001) (width 0.5) (layer B.Cu) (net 1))
 (segment (start 231.14 53.34) (end 220.98 53.34) (width 0.5) (layer B.Cu) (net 1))
 (segment (start 231.14 58.674) (end 231.14 58.42) (width 0.5) (layer B.Cu) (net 1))
 (segment (start 231.14 58.42) (end 231.14 57.912) (width 0.5) (layer B.Cu) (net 1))
 (segment (start 241.3 58.594) (end 231.314 58.594) (width 0.5) (layer B.Cu) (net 1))
 (segment (start 231.314 58.594) (end 231.14 58.42) (width 0.5) (layer B.Cu) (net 1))
 (segment (start 231.14 57.912) (end 231.14 53.34) (width 0.5) (layer B.Cu) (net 1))
 (segment (start 226.06 57.88) (end 231.108 57.88) (width 0.5) (layer B.Cu) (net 1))
 (segment (start 231.108 57.88) (end 231.14 57.912) (width 0.5) (layer B.Cu) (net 1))
 (segment (start 231.14 63.5) (end 231.14 58.674) (width 0.5) (layer B.Cu) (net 1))
 (segment (start 231.14 53.42) (end 231.22 53.34) (width 0.25) (layer B.Cu) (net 1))
 (segment (start 216.987001 59.872999) (end 213.33552 63.52448) (width 0.25) (layer B.Cu) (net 8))
 (segment (start 213.33552 63.52448) (end 205.73184 63.52448) (width 0.25) (layer B.Cu) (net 8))
 (segment (start 218.44 53.34) (end 216.987001 54.792999) (width 0.25) (layer B.Cu) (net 8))
 (segment (start 216.987001 54.792999) (end 216.987001 59.872999) (width 0.25) (layer B.Cu) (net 8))
 (segment (start 215.9 53.34) (end 215.9 52.07) (width 0.25) (layer B.Cu) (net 2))
 (segment (start 193.04 52.07) (end 193.04 54.61) (width 0.25) (layer B.Cu) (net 2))
 (segment (start 215.9 52.07) (end 214.63 50.8) (width 0.25) (layer B.Cu) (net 2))
 (segment (start 214.63 50.8) (end 194.31 50.8) (width 0.25) (layer B.Cu) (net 2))
 (segment (start 194.31 50.8) (end 193.04 52.07) (width 0.25) (layer B.Cu) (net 2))
 (segment (start 191.77 55.88) (end 190.5 55.88) (width 0.25) (layer B.Cu) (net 2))
 (segment (start 193.04 54.61) (end 191.77 55.88) (width 0.25) (layer B.Cu) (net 2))
 (segment (start 215.9 55.88) (end 215.9 57.0992) (width 0.25) (layer B.Cu) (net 5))
 (segment (start 215.9 57.0992) (end 214.5538 58.4454) (width 0.25) (layer B.Cu) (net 5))
 (segment (start 214.5538 58.4454) (end 214.55288 58.44448) (width 0.25) (layer B.Cu) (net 5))
 (segment (start 214.55288 58.44448) (end 205.73184 58.44448) (width 0.25) (layer B.Cu) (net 5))
 (segment (start 213.36 53.34) (end 206.8195 53.34) (width 0.25) (layer B.Cu) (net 3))
 (segment (start 205.73184 54.42766) (end 205.73184 55.90448) (width 0.25) (layer B.Cu) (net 3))
 (segment (start 206.8195 53.34) (end 205.73184 54.42766) (width 0.25) (layer B.Cu) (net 3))
 (segment (start 213.36 55.88) (end 214.63 54.61) (width 0.25) (layer B.Cu) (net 4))
 (segment (start 214.63 54.61) (end 214.63 52.07) (width 0.25) (layer B.Cu) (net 4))
 (segment (start 214.63 52.07) (end 203.2 52.07) (width 0.25) (layer B.Cu) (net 4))
 (segment (start 203.2 52.07) (end 201.93 53.34) (width 0.25) (layer B.Cu) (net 4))
 (segment (start 201.93 53.34) (end 201.93 80.01) (width 0.25) (layer B.Cu) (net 4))
 (segment (start 203.2 81.28) (end 205.74 81.28) (width 0.25) (layer B.Cu) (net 4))
 (segment (start 201.93 80.01) (end 203.2 81.28) (width 0.25) (layer B.Cu) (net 4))
 (segment (start 226.692 65.532) (end 228.6 65.532) (width 0.5) (layer B.Cu) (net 32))
 (segment (start 228.6 65.532) (end 232.918 65.532) (width 0.5) (layer B.Cu) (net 32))
 (segment (start 228.6 93.98) (end 228.6 65.532) (width 0.5) (layer B.Cu) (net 32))
 (segment (start 226.314 96.266) (end 228.6 93.98) (width 0.5) (layer B.Cu) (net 32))
 (segment (start 195.29336 96.266) (end 226.314 96.266) (width 0.5) (layer B.Cu) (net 32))
 (segment (start 190.49184 91.46448) (end 195.29336 96.266) (width 0.5) (layer B.Cu) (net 32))
 (segment (start 226.06 63.5) (end 226.06 64.9) (width 0.5) (layer B.Cu) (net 32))
 (segment (start 226.06 64.9) (end 226.692 65.532) (width 0.5) (layer B.Cu) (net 32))
 (segment (start 232.918 65.532) (end 233.68 64.77) (width 0.5) (layer B.Cu) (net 32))
 (segment (start 233.68 64.77) (end 233.68 63.5) (width 0.5) (layer B.Cu) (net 32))
 (segment (start 233.68 63.5) (end 241.827999 63.5) (width 0.5) (layer B.Cu) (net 32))
 (segment (start 241.827999 63.5) (end 243.078 62.249999) (width 0.5) (layer B.Cu) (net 32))
 (segment (start 241.827999 53.613999) (end 243.078 54.864) (width 0.5) (layer B.Cu) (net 32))
 (segment (start 243.078 54.824002) (end 243.078 62.23) (width 0.5) (layer B.Cu) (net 32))
 (segment (start 236.22 53.34) (end 241.046 53.34) (width 0.5) (layer B.Cu) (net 32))
 (segment (start 241.046 53.34) (end 241.3 53.594) (width 0.5) (layer B.Cu) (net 32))
 (segment (start 220.98 55.88) (end 222.05763 55.88) (width 0.5) (layer B.Cu) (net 7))
 (segment (start 222.05763 55.88) (end 226.06 55.88) (width 0.5) (layer B.Cu) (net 7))
 (segment (start 220.98 59.436) (end 220.98 55.88) (width 0.5) (layer B.Cu) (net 7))
 (segment (start 222.25 60.706) (end 220.98 59.436) (width 0.5) (layer B.Cu) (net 7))
 (segment (start 227.078792 60.706) (end 222.25 60.706) (width 0.5) (layer B.Cu) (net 7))
 (segment (start 228.6 63.5) (end 228.6 62.227208) (width 0.5) (layer B.Cu) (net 7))
 (segment (start 228.6 62.227208) (end 227.078792 60.706) (width 0.5) (layer B.Cu) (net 7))
 (segment (start 226.02 55.88) (end 226.06 55.92) (width 0.25) (layer B.Cu) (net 7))
 (segment (start 205.73184 60.98448) (end 204.36748 60.98448) (width 0.25) (layer B.Cu) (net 6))
 (segment (start 204.36748 60.98448) (end 204.343 60.96) (width 0.25) (layer B.Cu) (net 6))
 (segment (start 204.343 60.96) (end 203.327 61.976) (width 0.25) (layer B.Cu) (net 6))
 (segment (start 203.327 61.976) (end 203.327 63.881) (width 0.25) (layer B.Cu) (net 6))
 (segment (start 217.678001 56.641999) (end 218.44 55.88) (width 0.25) (layer B.Cu) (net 6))
 (segment (start 203.327 63.881) (end 204.343 64.897) (width 0.25) (layer B.Cu) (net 6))
 (segment (start 204.343 64.897) (end 216.408 64.897) (width 0.25) (layer B.Cu) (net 6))
 (segment (start 216.408 64.897) (end 217.678001 63.626999) (width 0.25) (layer B.Cu) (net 6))
 (segment (start 217.678001 63.626999) (end 217.678001 56.641999) (width 0.25) (layer B.Cu) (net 6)))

